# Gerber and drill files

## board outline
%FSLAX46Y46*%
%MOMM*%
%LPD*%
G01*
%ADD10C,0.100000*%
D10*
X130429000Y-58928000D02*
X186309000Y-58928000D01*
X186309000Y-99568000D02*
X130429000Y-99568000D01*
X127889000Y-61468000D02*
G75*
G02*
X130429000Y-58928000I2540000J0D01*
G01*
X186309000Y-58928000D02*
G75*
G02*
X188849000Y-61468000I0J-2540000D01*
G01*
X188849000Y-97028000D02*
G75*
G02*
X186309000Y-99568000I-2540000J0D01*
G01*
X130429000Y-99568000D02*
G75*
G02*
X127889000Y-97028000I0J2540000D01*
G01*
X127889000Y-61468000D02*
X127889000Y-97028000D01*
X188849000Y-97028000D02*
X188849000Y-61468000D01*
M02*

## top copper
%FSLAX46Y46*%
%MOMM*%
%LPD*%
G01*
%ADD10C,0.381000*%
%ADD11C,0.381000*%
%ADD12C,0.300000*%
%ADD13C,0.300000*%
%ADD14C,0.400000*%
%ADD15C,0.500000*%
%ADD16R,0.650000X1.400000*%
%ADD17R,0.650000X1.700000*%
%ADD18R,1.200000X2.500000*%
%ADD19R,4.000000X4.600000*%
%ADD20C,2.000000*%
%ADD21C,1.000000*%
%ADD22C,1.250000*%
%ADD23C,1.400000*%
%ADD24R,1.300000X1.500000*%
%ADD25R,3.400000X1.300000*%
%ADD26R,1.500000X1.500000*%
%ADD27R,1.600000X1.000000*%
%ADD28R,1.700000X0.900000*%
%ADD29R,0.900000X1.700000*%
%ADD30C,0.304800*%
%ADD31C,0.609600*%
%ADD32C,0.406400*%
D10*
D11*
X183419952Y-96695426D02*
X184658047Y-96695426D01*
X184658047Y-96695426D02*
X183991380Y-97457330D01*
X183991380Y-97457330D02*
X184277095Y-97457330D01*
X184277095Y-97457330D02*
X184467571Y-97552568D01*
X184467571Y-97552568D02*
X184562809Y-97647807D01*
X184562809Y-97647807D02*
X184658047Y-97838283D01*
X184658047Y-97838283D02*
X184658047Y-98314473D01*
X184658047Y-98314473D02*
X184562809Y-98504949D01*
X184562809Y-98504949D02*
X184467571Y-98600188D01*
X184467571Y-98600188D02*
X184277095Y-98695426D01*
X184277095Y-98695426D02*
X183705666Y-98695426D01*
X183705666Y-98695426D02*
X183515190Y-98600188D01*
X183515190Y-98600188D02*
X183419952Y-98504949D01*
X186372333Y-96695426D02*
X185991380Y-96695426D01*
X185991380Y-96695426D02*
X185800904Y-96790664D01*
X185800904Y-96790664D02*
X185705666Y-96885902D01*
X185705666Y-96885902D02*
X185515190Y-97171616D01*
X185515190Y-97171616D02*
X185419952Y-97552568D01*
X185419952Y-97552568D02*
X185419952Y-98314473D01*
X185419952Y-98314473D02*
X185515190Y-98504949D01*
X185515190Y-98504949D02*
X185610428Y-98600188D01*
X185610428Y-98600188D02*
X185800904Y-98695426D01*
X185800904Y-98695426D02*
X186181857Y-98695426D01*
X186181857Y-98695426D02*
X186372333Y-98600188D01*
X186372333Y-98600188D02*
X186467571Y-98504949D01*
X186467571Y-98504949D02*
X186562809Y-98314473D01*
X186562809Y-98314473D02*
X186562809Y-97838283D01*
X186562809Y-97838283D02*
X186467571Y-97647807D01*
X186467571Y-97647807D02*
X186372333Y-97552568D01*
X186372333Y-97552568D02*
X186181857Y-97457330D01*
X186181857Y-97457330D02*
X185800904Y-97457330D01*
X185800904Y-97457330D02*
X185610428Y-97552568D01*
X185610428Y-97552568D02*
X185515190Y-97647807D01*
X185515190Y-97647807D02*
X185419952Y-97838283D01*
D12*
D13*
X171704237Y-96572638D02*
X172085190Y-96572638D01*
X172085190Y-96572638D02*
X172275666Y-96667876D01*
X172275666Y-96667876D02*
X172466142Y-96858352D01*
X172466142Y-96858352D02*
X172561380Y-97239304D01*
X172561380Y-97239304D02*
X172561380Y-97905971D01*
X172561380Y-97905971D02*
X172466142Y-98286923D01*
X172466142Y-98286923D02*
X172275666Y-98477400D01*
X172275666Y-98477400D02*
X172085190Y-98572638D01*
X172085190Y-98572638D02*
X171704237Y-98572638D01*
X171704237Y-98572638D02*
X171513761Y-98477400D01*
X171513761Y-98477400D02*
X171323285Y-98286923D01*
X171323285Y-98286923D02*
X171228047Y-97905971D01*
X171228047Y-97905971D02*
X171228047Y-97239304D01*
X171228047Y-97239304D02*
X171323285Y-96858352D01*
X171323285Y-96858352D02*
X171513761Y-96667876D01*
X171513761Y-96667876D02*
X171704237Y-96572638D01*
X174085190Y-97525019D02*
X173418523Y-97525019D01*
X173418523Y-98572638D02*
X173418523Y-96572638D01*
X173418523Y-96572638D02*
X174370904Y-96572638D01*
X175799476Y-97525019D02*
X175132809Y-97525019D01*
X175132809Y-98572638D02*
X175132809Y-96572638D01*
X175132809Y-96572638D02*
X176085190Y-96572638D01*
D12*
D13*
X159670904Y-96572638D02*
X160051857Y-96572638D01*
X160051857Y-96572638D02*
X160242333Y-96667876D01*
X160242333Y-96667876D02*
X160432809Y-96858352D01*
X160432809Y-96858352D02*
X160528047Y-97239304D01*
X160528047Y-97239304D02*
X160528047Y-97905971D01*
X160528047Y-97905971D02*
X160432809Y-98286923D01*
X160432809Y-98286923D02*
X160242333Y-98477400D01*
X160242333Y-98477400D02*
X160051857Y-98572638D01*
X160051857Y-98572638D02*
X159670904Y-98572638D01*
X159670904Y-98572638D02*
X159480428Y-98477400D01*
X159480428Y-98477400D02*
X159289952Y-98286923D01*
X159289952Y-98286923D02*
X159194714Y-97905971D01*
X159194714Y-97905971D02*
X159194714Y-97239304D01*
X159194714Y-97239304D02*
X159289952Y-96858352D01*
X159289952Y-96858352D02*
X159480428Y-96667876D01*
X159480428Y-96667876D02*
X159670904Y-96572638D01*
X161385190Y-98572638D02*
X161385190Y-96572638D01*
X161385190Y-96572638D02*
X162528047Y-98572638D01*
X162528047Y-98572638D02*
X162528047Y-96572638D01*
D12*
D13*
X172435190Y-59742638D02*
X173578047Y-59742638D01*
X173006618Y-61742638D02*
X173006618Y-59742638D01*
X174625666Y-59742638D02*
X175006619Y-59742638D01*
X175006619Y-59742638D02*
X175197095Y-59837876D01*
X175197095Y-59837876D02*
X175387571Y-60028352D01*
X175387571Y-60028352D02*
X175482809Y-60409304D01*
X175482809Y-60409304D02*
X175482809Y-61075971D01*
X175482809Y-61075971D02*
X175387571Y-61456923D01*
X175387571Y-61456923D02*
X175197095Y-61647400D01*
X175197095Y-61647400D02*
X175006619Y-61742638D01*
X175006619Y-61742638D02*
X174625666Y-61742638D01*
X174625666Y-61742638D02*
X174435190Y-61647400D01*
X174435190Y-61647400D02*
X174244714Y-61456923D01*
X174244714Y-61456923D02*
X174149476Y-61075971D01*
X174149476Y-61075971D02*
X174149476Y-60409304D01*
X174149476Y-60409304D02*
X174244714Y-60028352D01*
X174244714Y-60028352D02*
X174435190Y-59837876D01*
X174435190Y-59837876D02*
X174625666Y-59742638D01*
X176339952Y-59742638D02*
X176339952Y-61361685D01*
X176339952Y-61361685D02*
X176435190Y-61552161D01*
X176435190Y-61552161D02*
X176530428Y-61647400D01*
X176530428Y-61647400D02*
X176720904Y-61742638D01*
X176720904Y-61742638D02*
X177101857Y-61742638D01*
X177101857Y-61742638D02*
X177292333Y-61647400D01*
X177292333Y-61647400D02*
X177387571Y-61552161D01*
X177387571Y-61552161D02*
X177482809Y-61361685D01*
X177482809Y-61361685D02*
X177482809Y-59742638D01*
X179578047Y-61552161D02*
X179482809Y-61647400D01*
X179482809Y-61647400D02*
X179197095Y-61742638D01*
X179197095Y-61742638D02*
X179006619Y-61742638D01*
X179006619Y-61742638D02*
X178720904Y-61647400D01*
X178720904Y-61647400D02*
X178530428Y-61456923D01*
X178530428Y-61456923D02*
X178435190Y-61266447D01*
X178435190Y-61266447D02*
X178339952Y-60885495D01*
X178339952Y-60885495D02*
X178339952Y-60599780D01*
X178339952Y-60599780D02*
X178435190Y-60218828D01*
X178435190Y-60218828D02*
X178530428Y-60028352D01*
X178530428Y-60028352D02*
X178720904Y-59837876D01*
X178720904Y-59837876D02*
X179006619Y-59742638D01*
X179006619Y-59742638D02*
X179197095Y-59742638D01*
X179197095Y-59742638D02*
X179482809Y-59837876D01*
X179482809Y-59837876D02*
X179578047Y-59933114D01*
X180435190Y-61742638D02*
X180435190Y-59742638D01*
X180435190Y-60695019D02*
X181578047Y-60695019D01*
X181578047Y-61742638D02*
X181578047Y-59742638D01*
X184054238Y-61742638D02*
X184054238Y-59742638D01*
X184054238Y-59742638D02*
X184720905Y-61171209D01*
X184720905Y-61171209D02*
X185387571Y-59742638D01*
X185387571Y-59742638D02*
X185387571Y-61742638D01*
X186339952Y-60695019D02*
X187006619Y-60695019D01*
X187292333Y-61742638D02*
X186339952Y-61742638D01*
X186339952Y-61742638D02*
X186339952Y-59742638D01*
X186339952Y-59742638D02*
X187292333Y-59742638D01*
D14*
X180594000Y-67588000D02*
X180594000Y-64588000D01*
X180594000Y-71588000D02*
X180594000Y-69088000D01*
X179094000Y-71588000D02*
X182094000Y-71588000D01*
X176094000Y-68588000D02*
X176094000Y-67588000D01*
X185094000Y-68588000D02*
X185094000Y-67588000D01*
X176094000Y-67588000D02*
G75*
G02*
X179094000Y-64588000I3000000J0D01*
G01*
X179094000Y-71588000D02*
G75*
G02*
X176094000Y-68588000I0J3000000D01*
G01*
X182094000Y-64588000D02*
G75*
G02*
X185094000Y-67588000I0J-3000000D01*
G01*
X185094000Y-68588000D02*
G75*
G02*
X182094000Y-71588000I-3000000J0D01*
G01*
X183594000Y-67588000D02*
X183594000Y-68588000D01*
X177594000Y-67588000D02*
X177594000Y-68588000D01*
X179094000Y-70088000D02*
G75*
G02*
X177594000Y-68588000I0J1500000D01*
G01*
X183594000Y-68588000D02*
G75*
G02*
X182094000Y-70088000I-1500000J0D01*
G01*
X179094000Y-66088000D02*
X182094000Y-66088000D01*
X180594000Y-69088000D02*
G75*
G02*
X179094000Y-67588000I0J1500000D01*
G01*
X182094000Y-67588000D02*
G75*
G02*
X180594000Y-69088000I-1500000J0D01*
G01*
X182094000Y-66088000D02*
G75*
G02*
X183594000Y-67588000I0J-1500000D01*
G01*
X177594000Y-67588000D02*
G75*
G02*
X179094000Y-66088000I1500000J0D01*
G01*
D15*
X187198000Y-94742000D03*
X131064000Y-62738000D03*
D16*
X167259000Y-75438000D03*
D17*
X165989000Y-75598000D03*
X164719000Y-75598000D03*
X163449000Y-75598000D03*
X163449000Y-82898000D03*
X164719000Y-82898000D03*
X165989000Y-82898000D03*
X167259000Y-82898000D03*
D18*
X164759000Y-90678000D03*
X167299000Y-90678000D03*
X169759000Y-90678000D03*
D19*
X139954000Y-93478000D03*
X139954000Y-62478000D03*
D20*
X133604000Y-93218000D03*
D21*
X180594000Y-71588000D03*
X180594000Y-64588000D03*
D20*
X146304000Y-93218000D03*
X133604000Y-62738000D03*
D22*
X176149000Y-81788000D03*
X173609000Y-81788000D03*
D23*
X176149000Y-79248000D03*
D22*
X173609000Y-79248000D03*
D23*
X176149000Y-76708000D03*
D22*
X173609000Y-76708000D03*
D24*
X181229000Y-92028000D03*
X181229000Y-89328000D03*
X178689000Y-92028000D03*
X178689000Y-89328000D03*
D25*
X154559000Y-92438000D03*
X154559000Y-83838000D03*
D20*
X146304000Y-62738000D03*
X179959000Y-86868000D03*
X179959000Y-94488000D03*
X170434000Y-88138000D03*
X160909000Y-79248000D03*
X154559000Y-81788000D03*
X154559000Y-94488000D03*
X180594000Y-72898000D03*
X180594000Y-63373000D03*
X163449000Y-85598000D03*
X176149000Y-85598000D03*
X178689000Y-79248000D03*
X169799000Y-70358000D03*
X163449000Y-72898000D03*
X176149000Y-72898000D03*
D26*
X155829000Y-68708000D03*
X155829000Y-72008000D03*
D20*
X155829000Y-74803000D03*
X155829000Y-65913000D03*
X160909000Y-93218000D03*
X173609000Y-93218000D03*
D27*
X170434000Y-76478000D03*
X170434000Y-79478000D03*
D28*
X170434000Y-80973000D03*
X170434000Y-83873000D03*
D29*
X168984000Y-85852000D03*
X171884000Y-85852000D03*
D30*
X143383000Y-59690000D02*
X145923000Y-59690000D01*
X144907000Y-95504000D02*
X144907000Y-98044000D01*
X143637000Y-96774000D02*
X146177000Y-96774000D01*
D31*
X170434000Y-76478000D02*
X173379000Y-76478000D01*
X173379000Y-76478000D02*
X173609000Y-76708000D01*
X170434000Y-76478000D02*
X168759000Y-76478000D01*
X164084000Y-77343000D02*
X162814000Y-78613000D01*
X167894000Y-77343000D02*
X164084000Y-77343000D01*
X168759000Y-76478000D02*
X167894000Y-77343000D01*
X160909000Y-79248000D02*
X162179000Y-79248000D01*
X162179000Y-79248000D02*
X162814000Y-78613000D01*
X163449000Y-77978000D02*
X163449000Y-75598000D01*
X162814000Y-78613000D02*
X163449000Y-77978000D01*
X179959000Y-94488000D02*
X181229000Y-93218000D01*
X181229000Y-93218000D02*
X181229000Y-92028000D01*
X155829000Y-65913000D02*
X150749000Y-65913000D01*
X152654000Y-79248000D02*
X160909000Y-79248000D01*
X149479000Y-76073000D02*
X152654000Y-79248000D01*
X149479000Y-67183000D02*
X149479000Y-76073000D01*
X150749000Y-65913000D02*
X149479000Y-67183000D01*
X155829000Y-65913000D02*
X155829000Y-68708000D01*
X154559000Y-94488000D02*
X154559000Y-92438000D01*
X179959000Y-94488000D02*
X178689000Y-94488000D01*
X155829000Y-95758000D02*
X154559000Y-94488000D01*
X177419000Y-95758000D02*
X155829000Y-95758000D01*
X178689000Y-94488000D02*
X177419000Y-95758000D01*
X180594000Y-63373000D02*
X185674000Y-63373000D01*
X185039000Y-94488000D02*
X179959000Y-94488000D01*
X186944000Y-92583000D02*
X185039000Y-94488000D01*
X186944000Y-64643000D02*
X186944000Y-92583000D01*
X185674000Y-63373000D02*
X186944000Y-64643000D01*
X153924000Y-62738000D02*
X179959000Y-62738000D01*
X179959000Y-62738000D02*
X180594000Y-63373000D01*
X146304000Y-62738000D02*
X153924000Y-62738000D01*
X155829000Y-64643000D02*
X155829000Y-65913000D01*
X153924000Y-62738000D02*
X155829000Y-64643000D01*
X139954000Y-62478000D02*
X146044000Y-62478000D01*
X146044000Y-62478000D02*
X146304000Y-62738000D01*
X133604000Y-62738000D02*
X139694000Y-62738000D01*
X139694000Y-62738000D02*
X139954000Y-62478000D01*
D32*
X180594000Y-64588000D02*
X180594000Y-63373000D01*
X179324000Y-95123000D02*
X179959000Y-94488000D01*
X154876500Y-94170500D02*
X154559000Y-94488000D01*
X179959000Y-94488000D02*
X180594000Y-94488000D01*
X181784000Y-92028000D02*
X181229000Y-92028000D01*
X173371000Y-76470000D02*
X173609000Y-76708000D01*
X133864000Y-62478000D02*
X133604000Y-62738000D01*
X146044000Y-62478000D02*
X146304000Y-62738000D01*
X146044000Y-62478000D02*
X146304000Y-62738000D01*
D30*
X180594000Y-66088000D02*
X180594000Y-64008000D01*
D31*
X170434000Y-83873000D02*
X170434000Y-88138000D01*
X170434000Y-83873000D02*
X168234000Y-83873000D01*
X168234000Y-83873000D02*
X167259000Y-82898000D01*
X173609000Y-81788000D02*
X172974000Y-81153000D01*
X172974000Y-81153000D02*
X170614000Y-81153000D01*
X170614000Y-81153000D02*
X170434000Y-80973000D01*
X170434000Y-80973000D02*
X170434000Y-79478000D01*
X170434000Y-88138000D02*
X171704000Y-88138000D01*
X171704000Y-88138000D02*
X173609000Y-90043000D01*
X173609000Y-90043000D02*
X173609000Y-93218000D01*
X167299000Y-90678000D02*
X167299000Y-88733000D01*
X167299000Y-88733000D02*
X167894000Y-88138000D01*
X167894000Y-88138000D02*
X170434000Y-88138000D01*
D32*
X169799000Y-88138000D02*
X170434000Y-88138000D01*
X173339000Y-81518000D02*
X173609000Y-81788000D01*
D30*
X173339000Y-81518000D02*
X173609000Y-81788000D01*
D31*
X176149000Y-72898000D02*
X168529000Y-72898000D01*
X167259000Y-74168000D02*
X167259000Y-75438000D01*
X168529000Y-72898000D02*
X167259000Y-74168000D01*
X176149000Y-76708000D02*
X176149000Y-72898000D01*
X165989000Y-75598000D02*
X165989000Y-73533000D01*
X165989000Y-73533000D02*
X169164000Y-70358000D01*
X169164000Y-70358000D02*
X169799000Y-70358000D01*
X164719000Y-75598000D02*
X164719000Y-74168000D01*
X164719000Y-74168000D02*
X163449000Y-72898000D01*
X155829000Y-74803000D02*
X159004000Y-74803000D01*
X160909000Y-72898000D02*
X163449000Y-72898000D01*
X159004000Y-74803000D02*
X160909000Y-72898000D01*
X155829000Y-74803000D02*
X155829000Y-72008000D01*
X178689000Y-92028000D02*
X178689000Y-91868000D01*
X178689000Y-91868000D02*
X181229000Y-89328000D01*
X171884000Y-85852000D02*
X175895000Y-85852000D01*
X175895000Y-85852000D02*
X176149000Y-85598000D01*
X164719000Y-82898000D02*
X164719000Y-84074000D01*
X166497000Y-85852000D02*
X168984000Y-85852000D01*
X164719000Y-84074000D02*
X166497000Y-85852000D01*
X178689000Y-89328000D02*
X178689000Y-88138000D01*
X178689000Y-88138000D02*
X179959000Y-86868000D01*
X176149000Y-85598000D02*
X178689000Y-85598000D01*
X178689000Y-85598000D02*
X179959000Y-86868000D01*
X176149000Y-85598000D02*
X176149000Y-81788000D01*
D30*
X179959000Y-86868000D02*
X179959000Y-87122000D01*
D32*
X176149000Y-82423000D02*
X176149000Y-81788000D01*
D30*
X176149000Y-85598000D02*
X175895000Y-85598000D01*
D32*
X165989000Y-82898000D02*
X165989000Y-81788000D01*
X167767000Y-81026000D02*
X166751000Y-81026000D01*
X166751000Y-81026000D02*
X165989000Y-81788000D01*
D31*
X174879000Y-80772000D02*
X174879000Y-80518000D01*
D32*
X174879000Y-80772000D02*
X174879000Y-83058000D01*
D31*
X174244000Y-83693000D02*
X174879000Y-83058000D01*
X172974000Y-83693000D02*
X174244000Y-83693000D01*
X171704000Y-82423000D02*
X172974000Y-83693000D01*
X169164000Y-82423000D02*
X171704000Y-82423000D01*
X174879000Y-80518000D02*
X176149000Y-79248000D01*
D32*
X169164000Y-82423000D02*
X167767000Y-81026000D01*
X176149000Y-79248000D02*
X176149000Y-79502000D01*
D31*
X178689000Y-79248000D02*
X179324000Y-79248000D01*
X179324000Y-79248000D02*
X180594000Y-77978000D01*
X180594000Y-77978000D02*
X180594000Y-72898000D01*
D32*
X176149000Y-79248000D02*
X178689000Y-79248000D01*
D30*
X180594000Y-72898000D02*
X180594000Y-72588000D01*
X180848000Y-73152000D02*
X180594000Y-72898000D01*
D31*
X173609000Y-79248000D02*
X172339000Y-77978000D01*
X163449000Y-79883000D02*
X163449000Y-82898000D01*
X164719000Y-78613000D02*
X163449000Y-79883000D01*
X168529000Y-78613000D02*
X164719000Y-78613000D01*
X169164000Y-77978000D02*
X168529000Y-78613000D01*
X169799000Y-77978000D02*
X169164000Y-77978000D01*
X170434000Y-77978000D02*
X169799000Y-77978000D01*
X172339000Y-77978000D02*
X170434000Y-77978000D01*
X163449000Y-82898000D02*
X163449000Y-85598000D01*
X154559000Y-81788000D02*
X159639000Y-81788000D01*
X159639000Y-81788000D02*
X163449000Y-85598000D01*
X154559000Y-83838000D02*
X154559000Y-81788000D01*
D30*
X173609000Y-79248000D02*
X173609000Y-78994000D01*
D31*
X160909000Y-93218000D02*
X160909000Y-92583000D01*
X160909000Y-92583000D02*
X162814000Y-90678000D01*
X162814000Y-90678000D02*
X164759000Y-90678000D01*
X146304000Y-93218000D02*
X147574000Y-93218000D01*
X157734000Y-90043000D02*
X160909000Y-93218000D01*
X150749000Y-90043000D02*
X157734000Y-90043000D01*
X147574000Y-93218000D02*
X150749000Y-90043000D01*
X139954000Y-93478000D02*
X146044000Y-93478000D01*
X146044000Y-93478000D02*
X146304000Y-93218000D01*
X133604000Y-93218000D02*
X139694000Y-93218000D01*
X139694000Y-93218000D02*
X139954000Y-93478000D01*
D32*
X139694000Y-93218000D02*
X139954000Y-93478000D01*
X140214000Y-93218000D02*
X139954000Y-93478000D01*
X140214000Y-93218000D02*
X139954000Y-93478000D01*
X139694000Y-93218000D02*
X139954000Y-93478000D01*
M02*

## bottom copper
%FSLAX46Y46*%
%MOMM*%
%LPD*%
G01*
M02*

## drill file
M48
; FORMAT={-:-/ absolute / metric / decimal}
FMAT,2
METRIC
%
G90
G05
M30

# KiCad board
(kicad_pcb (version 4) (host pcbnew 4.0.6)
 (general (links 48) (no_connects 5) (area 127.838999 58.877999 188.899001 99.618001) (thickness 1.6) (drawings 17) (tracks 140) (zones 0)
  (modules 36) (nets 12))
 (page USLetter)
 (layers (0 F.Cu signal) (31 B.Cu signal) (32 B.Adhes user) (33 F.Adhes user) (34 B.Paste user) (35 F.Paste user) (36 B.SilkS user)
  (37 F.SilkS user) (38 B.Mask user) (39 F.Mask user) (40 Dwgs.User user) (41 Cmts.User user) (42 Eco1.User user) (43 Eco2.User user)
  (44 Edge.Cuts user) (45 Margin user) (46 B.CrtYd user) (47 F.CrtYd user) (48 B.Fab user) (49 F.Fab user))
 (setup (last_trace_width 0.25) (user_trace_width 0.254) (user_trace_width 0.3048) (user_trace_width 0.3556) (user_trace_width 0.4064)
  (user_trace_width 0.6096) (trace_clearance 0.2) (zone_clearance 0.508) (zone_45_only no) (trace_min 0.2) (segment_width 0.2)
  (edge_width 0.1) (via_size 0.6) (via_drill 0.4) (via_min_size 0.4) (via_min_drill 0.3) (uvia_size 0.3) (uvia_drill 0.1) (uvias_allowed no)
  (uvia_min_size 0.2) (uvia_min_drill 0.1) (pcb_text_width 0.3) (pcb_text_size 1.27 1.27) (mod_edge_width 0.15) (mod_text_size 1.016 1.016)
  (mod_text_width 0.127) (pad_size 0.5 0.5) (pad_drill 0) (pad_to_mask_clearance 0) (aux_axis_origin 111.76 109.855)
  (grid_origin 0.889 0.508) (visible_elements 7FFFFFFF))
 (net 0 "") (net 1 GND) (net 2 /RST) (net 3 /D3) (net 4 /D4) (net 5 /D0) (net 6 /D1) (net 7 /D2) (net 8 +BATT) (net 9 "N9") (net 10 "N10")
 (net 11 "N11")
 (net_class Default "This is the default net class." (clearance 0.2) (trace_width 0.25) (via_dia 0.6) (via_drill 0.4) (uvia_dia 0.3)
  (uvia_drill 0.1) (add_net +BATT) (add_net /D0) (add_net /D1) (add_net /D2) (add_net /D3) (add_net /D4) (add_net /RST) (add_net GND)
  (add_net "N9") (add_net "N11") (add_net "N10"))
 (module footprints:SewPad (layer F.Cu) (at 187.198 94.742)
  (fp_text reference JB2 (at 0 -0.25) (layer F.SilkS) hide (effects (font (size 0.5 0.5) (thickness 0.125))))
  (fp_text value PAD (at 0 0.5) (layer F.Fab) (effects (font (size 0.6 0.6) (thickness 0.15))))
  (pad 1 smd circle (at 0 0) (size 0.5 0.5) (layers F.Cu F.Mask) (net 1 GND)))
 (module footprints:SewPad (layer F.Cu) (at 131.064 62.738)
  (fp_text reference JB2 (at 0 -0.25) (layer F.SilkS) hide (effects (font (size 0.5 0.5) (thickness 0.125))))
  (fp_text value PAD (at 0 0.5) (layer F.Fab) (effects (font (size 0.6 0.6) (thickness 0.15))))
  (pad 1 smd circle (at 0 0) (size 0.5 0.5) (layers F.Cu F.Mask) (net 1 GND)))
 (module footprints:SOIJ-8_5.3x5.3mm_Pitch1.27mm (layer F.Cu) (at 165.354 79.248 270)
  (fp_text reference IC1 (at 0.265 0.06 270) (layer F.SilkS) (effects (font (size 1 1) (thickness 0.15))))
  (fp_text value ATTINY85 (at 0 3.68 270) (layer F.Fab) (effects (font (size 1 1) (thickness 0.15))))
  (pad 1 smd rect (at -3.81 -1.905 270) (size 1.4 0.65) (layers F.Cu F.Paste F.Mask) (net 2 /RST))
  (pad 2 smd rect (at -3.65 -0.635 270) (size 1.7 0.65) (layers F.Cu F.Paste F.Mask) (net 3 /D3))
  (pad 3 smd rect (at -3.65 0.635 270) (size 1.7 0.65) (layers F.Cu F.Paste F.Mask) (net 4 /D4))
  (pad 4 smd rect (at -3.65 1.905 270) (size 1.7 0.65) (layers F.Cu F.Paste F.Mask) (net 1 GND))
  (pad 5 smd rect (at 3.65 1.905 270) (size 1.7 0.65) (layers F.Cu F.Paste F.Mask) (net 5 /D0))
  (pad 6 smd rect (at 3.65 0.635 270) (size 1.7 0.65) (layers F.Cu F.Paste F.Mask) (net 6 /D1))
  (pad 7 smd rect (at 3.65 -0.635 270) (size 1.7 0.65) (layers F.Cu F.Paste F.Mask) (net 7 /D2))
  (pad 8 smd rect (at 3.65 -1.905 270) (size 1.7 0.65) (layers F.Cu F.Paste F.Mask) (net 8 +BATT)))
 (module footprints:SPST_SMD (layer F.Cu) (at 167.259 90.678)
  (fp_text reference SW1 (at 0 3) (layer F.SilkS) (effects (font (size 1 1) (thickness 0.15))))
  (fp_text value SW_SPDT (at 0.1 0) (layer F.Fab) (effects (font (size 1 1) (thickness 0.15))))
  (pad 1 smd rect (at -2.5 0) (size 1.2 2.5) (layers F.Cu F.Paste F.Mask) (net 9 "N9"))
  (pad 2 smd rect (at 0.04 0) (size 1.2 2.5) (layers F.Cu F.Paste F.Mask) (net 8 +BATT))
  (pad 3 smd rect (at 2.5 0) (size 1.2 2.5) (layers F.Cu F.Paste F.Mask) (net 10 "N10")))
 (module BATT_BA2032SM (layer F.Cu) (at 139.954 77.978 90)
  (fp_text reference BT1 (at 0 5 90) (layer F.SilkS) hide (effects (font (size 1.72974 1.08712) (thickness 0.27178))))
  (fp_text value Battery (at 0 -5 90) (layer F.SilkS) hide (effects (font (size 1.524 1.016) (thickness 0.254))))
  (pad 1 smd rect (at -15.5 0 90) (size 4.6 4) (layers F.Cu F.Paste F.Mask) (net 9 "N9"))
  (pad 2 smd rect (at 15.5 0 90) (size 4.6 4) (layers F.Cu F.Paste F.Mask) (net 1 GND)))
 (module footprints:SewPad (layer F.Cu) (at 133.604 93.218)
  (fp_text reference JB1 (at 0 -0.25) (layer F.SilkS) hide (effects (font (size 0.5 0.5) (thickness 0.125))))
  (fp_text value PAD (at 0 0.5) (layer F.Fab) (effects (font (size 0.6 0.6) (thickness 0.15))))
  (pad 1 smd circle (at 0 0) (size 2 2) (layers F.Cu F.Mask) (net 9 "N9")))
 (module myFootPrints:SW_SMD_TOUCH (layer F.Cu) (at 180.594 69.088)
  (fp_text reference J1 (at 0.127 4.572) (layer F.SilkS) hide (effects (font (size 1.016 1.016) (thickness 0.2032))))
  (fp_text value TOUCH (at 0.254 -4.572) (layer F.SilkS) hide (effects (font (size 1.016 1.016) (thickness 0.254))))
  (fp_line (start 0 -1.5) (end 0 -4.5) (layer F.Cu) (width 0.4)) (fp_line (start 0 2.5) (end 0 0) (layer F.Cu) (width 0.4))
  (fp_line (start -1.5 2.5) (end 1.5 2.5) (layer F.Cu) (width 0.4))
  (fp_line (start -4.5 -0.5) (end -4.5 -1.5) (layer F.Cu) (width 0.4))
  (fp_line (start 4.5 -0.5) (end 4.5 -1.5) (layer F.Cu) (width 0.4))
  (fp_arc (start -1.5 -1.5) (end -4.5 -1.5) (angle 90) (layer F.Cu) (width 0.4))
  (fp_arc (start -1.5 -0.5) (end -1.5 2.5) (angle 90) (layer F.Cu) (width 0.4))
  (fp_arc (start 1.5 -1.5) (end 1.5 -4.5) (angle 90) (layer F.Cu) (width 0.4))
  (fp_arc (start 1.5 -0.5) (end 4.5 -0.5) (angle 90) (layer F.Cu) (width 0.4))
  (fp_line (start 3 -1.5) (end 3 -0.5) (layer F.Cu) (width 0.4))
  (fp_line (start -3 -1.5) (end -3 -0.5) (layer F.Cu) (width 0.4))
  (fp_arc (start -1.5 -0.5) (end -1.5 1) (angle 90) (layer F.Cu) (width 0.4))
  (fp_arc (start 1.5 -0.5) (end 3 -0.5) (angle 90) (layer F.Cu) (width 0.4))
  (fp_line (start -1.5 -3) (end 1.5 -3) (layer F.Cu) (width 0.4))
  (fp_arc (start 0 -1.5) (end 0 0) (angle 90) (layer F.Cu) (width 0.4))
  (fp_arc (start 0 -1.5) (end 1.5 -1.5) (angle 90) (layer F.Cu) (width 0.4))
  (fp_arc (start 1.5 -1.5) (end 1.5 -3) (angle 90) (layer F.Cu) (width 0.4))
  (fp_arc (start -1.5 -1.5) (end -3 -1.5) (angle 90) (layer F.Cu) (width 0.4))
  (pad 2 smd circle (at 0 2.5) (size 1 1) (layers F.Cu) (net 7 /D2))
  (pad 1 smd circle (at 0 -4.5) (size 1 1) (layers F.Cu) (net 1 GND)))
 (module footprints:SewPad (layer F.Cu) (at 146.304 93.218)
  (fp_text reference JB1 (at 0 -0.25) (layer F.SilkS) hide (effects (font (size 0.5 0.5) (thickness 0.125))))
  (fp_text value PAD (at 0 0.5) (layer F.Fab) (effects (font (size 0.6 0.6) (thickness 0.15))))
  (pad 1 smd circle (at 0 0) (size 2 2) (layers F.Cu F.Mask) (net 9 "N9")))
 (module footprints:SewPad (layer F.Cu) (at 133.604 62.738)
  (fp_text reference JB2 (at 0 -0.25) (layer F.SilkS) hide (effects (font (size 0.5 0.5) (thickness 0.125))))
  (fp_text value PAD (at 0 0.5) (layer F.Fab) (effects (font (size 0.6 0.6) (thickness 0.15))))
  (pad 1 smd circle (at 0 0) (size 2 2) (layers F.Cu F.Mask) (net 1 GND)))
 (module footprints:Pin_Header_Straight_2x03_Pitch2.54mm (layer F.Cu) (at 176.149 81.788 180)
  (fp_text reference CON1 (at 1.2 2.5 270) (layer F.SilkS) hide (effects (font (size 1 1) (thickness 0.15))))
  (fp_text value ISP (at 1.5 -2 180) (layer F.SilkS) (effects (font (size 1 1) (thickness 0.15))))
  (pad 1 smd circle (at 0 0 180) (size 1.25 1.25) (layers F.Cu) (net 6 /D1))
  (pad 2 smd circle (at 2.54 0 180) (size 1.25 1.25) (layers F.Cu) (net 8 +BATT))
  (pad 3 smd circle (at 0 2.54 180) (size 1.4 1.4) (layers F.Cu) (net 7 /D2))
  (pad 4 smd circle (at 2.54 2.54 180) (size 1.25 1.25) (layers F.Cu) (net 5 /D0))
  (pad 5 smd circle (at 0 5.08 180) (size 1.4 1.4) (layers F.Cu) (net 2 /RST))
  (pad 6 smd circle (at 2.54 5.08 180) (size 1.25 1.25) (layers F.Cu) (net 1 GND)))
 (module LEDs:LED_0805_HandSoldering (layer F.Cu) (at 181.229 90.678 90)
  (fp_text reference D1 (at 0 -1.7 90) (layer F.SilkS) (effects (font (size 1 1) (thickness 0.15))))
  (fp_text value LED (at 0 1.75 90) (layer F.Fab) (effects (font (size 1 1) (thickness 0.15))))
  (pad 1 smd rect (at -1.35 0 90) (size 1.5 1.3) (layers F.Cu F.Paste F.Mask) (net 1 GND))
  (pad 2 smd rect (at 1.35 0 90) (size 1.5 1.3) (layers F.Cu F.Paste F.Mask) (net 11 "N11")))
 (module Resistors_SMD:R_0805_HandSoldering (layer F.Cu) (at 178.689 90.678 90)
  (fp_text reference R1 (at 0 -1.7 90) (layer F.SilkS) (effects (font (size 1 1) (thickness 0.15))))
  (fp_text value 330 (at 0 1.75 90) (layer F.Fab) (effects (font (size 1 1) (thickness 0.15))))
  (pad 1 smd rect (at -1.35 0 90) (size 1.5 1.3) (layers F.Cu F.Paste F.Mask) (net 11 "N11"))
  (pad 2 smd rect (at 1.35 0 90) (size 1.5 1.3) (layers F.Cu F.Paste F.Mask) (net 6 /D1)))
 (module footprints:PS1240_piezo (layer F.Cu) (at 154.559 88.138 90)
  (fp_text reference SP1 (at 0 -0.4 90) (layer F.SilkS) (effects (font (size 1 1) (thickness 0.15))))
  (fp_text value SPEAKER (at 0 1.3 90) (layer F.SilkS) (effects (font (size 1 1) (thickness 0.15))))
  (pad 1 smd rect (at -4.3 0 90) (size 1.3 3.4) (layers F.Cu F.Paste F.Mask) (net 1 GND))
  (pad 2 smd rect (at 4.3 0 90) (size 1.3 3.4) (layers F.Cu F.Paste F.Mask) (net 5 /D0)))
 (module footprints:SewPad (layer F.Cu) (at 146.304 62.738)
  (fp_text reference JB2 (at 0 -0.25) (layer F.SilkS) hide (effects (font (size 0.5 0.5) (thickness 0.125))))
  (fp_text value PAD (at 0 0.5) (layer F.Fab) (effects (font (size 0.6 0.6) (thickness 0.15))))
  (pad 1 smd circle (at 0 0) (size 2 2) (layers F.Cu F.Mask) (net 1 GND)))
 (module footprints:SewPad (layer F.Cu) (at 179.959 86.868 90)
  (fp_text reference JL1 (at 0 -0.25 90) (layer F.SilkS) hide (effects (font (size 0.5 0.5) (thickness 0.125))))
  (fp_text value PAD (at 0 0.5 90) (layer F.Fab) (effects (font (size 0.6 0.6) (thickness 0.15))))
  (pad 1 smd circle (at 0 0 90) (size 2 2) (layers F.Cu F.Mask) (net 6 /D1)))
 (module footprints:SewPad (layer F.Cu) (at 179.959 94.488 90)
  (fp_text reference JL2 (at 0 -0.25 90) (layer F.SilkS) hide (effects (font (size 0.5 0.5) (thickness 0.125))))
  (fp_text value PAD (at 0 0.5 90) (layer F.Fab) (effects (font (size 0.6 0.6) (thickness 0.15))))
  (pad 1 smd circle (at 0 0 90) (size 2 2) (layers F.Cu F.Mask) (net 1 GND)))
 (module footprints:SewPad (layer F.Cu) (at 170.434 88.138)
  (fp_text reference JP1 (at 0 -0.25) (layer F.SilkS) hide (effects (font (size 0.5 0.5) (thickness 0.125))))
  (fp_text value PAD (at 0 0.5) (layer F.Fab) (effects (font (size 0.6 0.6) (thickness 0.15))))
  (pad 1 smd circle (at 0 0) (size 2 2) (layers F.Cu F.Mask) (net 8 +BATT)))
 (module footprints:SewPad (layer F.Cu) (at 160.909 79.248)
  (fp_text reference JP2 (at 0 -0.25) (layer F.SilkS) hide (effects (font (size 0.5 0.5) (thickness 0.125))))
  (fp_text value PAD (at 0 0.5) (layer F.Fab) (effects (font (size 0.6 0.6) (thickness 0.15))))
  (pad 1 smd circle (at 0 0) (size 2 2) (layers F.Cu F.Mask) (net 1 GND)))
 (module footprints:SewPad (layer F.Cu) (at 154.559 81.788 180)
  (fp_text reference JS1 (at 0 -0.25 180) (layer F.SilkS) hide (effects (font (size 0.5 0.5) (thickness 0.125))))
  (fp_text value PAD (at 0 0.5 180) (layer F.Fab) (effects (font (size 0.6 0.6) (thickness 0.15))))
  (pad 1 smd circle (at 0 0 180) (size 2 2) (layers F.Cu F.Mask) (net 5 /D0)))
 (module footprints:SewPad (layer F.Cu) (at 154.559 94.488 180)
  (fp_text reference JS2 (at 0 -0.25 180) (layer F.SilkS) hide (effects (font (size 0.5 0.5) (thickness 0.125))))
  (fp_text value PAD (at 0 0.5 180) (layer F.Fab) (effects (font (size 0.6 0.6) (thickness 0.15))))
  (pad 1 smd circle (at 0 0 180) (size 2 2) (layers F.Cu F.Mask) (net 1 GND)))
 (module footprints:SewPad (layer F.Cu) (at 180.594 72.898 90)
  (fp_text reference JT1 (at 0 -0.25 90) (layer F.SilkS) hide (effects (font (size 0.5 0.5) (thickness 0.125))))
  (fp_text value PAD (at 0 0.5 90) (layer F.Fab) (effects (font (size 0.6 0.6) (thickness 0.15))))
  (pad 1 smd circle (at 0 0 90) (size 2 2) (layers F.Cu F.Mask) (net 7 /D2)))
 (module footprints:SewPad (layer F.Cu) (at 180.594 63.373 90)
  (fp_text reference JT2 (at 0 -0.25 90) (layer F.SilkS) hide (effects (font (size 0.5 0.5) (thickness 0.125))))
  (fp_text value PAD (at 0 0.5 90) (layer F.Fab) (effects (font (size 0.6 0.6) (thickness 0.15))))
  (pad 1 smd circle (at 0 0 90) (size 2 2) (layers F.Cu F.Mask) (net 1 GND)))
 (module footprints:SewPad (layer F.Cu) (at 163.449 85.598)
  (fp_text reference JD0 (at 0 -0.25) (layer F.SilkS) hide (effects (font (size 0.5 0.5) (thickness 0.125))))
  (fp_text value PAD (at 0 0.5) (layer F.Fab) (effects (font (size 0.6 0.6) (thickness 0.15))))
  (pad 1 smd circle (at 0 0) (size 2 2) (layers F.Cu F.Mask) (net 5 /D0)))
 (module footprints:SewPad (layer F.Cu) (at 176.149 85.598)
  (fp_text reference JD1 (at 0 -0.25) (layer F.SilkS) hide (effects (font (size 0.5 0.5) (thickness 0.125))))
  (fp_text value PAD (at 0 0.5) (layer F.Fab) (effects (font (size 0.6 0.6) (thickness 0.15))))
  (pad 1 smd circle (at 0 0) (size 2 2) (layers F.Cu F.Mask) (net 6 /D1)))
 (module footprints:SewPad (layer F.Cu) (at 178.689 79.248)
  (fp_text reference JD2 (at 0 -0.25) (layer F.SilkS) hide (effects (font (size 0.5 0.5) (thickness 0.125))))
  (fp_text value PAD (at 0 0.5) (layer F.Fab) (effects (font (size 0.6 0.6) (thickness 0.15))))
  (pad 1 smd circle (at 0 0) (size 2 2) (layers F.Cu F.Mask) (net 7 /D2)))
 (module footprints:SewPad (layer F.Cu) (at 169.799 70.358)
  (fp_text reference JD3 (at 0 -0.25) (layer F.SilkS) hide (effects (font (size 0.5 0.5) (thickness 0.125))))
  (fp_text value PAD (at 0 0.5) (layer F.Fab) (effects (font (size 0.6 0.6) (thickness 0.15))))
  (pad 1 smd circle (at 0 0) (size 2 2) (layers F.Cu F.Mask) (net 3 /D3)))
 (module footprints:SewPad (layer F.Cu) (at 163.449 72.898)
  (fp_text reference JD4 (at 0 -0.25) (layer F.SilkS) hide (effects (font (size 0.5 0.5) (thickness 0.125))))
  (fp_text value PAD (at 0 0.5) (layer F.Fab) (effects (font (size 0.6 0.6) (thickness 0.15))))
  (pad 1 smd circle (at 0 0) (size 2 2) (layers F.Cu F.Mask) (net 4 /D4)))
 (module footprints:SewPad (layer F.Cu) (at 176.149 72.898)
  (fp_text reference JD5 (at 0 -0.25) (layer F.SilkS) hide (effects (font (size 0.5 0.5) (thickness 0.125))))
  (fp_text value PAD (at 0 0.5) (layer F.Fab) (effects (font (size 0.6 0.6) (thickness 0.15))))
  (pad 1 smd circle (at 0 0) (size 2 2) (layers F.Cu F.Mask) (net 2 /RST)))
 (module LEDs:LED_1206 (layer F.Cu) (at 155.829 70.358 90)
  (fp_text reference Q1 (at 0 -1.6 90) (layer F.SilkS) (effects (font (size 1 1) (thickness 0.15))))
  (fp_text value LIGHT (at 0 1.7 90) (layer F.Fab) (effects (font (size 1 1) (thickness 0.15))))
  (pad 2 smd rect (at 1.65 0 270) (size 1.5 1.5) (layers F.Cu F.Paste F.Mask) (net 1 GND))
  (pad 1 smd rect (at -1.65 0 270) (size 1.5 1.5) (layers F.Cu F.Paste F.Mask) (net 4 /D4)))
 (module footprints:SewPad (layer F.Cu) (at 155.829 74.803)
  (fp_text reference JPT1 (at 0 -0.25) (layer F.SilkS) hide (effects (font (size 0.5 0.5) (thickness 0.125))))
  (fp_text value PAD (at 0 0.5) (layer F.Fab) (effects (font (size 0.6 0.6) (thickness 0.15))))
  (pad 1 smd circle (at 0 0) (size 2 2) (layers F.Cu F.Mask) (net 4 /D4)))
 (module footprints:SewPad (layer F.Cu) (at 155.829 65.913)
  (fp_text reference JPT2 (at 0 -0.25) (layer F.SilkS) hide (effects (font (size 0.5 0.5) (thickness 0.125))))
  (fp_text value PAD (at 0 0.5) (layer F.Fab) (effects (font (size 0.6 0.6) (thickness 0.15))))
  (pad 1 smd circle (at 0 0) (size 2 2) (layers F.Cu F.Mask) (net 1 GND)))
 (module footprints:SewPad (layer F.Cu) (at 160.909 93.218)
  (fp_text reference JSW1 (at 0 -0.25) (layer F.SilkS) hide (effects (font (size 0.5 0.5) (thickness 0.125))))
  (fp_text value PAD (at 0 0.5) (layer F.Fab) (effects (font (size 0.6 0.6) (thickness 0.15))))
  (pad 1 smd circle (at 0 0) (size 2 2) (layers F.Cu F.Mask) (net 9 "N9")))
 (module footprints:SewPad (layer F.Cu) (at 173.609 93.218)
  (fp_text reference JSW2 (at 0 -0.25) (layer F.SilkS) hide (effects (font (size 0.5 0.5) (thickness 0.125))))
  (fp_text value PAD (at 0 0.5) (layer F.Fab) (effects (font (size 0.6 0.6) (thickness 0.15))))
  (pad 1 smd circle (at 0 0) (size 2 2) (layers F.Cu F.Mask) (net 8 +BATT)))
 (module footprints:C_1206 (layer F.Cu) (at 170.434 77.978 270)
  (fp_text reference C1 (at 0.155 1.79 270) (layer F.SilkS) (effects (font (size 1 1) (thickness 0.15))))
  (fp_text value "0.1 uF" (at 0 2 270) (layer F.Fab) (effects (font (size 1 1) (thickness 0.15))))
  (pad 1 smd rect (at -1.5 0 270) (size 1 1.6) (layers F.Cu F.Paste F.Mask) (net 1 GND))
  (pad 2 smd rect (at 1.5 0 270) (size 1 1.6) (layers F.Cu F.Paste F.Mask) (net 8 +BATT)))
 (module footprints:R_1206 (layer F.Cu) (at 170.434 82.423 270)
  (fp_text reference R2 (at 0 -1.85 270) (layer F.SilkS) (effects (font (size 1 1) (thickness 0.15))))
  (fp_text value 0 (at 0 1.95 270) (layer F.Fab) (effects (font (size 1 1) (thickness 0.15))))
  (pad 1 smd rect (at -1.45 0 270) (size 0.9 1.7) (layers F.Cu F.Paste F.Mask) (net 8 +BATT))
  (pad 2 smd rect (at 1.45 0 270) (size 0.9 1.7) (layers F.Cu F.Paste F.Mask) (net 8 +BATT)))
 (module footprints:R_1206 (layer F.Cu) (at 170.434 85.852)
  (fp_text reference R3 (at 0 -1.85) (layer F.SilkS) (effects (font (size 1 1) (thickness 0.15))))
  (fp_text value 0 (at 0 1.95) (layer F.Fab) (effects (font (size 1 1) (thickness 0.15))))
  (pad 1 smd rect (at -1.45 0) (size 0.9 1.7) (layers F.Cu F.Paste F.Mask) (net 6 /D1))
  (pad 2 smd rect (at 1.45 0) (size 0.9 1.7) (layers F.Cu F.Paste F.Mask) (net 6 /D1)))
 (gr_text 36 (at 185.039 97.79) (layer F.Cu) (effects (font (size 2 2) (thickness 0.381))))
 (gr_line (start 130.429 58.928) (end 186.309 58.928) (angle 90) (layer Edge.Cuts) (width 0.1))
 (gr_line (start 186.309 99.568) (end 130.429 99.568) (angle 90) (layer Edge.Cuts) (width 0.1))
 (gr_arc (start 130.429 61.468) (end 127.889 61.468) (angle 90) (layer Edge.Cuts) (width 0.1))
 (gr_arc (start 186.309 61.468) (end 186.309 58.928) (angle 90) (layer Edge.Cuts) (width 0.1))
 (gr_arc (start 186.309 97.028) (end 188.849 97.028) (angle 90) (layer Edge.Cuts) (width 0.1))
 (gr_arc (start 130.429 97.028) (end 130.429 99.568) (angle 90) (layer Edge.Cuts) (width 0.1))
 (gr_line (start 127.889 61.468) (end 127.889 97.028) (angle 90) (layer Edge.Cuts) (width 0.1))
 (gr_line (start 188.849 97.028) (end 188.849 61.468) (angle 90) (layer Edge.Cuts) (width 0.1))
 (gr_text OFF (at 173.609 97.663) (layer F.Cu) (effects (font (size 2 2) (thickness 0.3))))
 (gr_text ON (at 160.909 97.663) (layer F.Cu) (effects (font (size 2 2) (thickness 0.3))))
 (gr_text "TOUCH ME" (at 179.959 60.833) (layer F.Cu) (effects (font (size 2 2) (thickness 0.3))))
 (segment (start 143.383 59.69) (end 145.923 59.69) (width 0.3048) (layer F.Cu) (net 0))
 (segment (start 144.907 95.504) (end 144.907 98.044) (width 0.3048) (layer F.Cu) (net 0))
 (segment (start 143.637 96.774) (end 146.177 96.774) (width 0.3048) (layer F.Cu) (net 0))
 (segment (start 170.434 76.478) (end 173.379 76.478) (width 0.6096) (layer F.Cu) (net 1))
 (segment (start 173.379 76.478) (end 173.609 76.708) (width 0.6096) (layer F.Cu) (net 1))
 (segment (start 170.434 76.478) (end 168.759 76.478) (width 0.6096) (layer F.Cu) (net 1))
 (segment (start 164.084 77.343) (end 162.814 78.613) (width 0.6096) (layer F.Cu) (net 1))
 (segment (start 167.894 77.343) (end 164.084 77.343) (width 0.6096) (layer F.Cu) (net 1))
 (segment (start 168.759 76.478) (end 167.894 77.343) (width 0.6096) (layer F.Cu) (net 1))
 (segment (start 160.909 79.248) (end 162.179 79.248) (width 0.6096) (layer F.Cu) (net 1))
 (segment (start 162.179 79.248) (end 162.814 78.613) (width 0.6096) (layer F.Cu) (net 1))
 (segment (start 163.449 77.978) (end 163.449 75.598) (width 0.6096) (layer F.Cu) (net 1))
 (segment (start 162.814 78.613) (end 163.449 77.978) (width 0.6096) (layer F.Cu) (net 1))
 (segment (start 179.959 94.488) (end 181.229 93.218) (width 0.6096) (layer F.Cu) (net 1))
 (segment (start 181.229 93.218) (end 181.229 92.028) (width 0.6096) (layer F.Cu) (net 1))
 (segment (start 155.829 65.913) (end 150.749 65.913) (width 0.6096) (layer F.Cu) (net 1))
 (segment (start 152.654 79.248) (end 160.909 79.248) (width 0.6096) (layer F.Cu) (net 1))
 (segment (start 149.479 76.073) (end 152.654 79.248) (width 0.6096) (layer F.Cu) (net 1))
 (segment (start 149.479 67.183) (end 149.479 76.073) (width 0.6096) (layer F.Cu) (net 1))
 (segment (start 150.749 65.913) (end 149.479 67.183) (width 0.6096) (layer F.Cu) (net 1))
 (segment (start 155.829 65.913) (end 155.829 68.708) (width 0.6096) (layer F.Cu) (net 1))
 (segment (start 154.559 94.488) (end 154.559 92.438) (width 0.6096) (layer F.Cu) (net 1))
 (segment (start 179.959 94.488) (end 178.689 94.488) (width 0.6096) (layer F.Cu) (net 1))
 (segment (start 155.829 95.758) (end 154.559 94.488) (width 0.6096) (layer F.Cu) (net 1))
 (segment (start 177.419 95.758) (end 155.829 95.758) (width 0.6096) (layer F.Cu) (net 1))
 (segment (start 178.689 94.488) (end 177.419 95.758) (width 0.6096) (layer F.Cu) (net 1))
 (segment (start 180.594 63.373) (end 185.674 63.373) (width 0.6096) (layer F.Cu) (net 1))
 (segment (start 185.039 94.488) (end 179.959 94.488) (width 0.6096) (layer F.Cu) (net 1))
 (segment (start 186.944 92.583) (end 185.039 94.488) (width 0.6096) (layer F.Cu) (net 1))
 (segment (start 186.944 64.643) (end 186.944 92.583) (width 0.6096) (layer F.Cu) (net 1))
 (segment (start 185.674 63.373) (end 186.944 64.643) (width 0.6096) (layer F.Cu) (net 1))
 (segment (start 153.924 62.738) (end 179.959 62.738) (width 0.6096) (layer F.Cu) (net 1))
 (segment (start 179.959 62.738) (end 180.594 63.373) (width 0.6096) (layer F.Cu) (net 1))
 (segment (start 146.304 62.738) (end 153.924 62.738) (width 0.6096) (layer F.Cu) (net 1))
 (segment (start 155.829 64.643) (end 155.829 65.913) (width 0.6096) (layer F.Cu) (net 1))
 (segment (start 153.924 62.738) (end 155.829 64.643) (width 0.6096) (layer F.Cu) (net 1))
 (segment (start 139.954 62.478) (end 146.044 62.478) (width 0.6096) (layer F.Cu) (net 1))
 (segment (start 146.044 62.478) (end 146.304 62.738) (width 0.6096) (layer F.Cu) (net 1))
 (segment (start 133.604 62.738) (end 139.694 62.738) (width 0.6096) (layer F.Cu) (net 1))
 (segment (start 139.694 62.738) (end 139.954 62.478) (width 0.6096) (layer F.Cu) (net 1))
 (segment (start 180.594 64.588) (end 180.594 63.373) (width 0.4064) (layer F.Cu) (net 1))
 (segment (start 179.324 95.123) (end 179.959 94.488) (width 0.4064) (layer F.Cu) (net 1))
 (segment (start 154.8765 94.1705) (end 154.559 94.488) (width 0.4064) (layer F.Cu) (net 1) (status 30))
 (segment (start 179.959 94.488) (end 180.594 94.488) (width 0.4064) (layer F.Cu) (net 1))
 (segment (start 181.784 92.028) (end 181.229 92.028) (width 0.4064) (layer F.Cu) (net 1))
 (segment (start 173.371 76.47) (end 173.609 76.708) (width 0.4064) (layer F.Cu) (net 1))
 (segment (start 133.864 62.478) (end 133.604 62.738) (width 0.4064) (layer F.Cu) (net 1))
 (segment (start 146.044 62.478) (end 146.304 62.738) (width 0.4064) (layer F.Cu) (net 1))
 (segment (start 146.044 62.478) (end 146.304 62.738) (width 0.4064) (layer F.Cu) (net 1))
 (segment (start 180.594 66.088) (end 180.594 64.008) (width 0.3048) (layer F.Cu) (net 1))
 (segment (start 170.434 83.873) (end 170.434 88.138) (width 0.6096) (layer F.Cu) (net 8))
 (segment (start 170.434 83.873) (end 168.234 83.873) (width 0.6096) (layer F.Cu) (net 8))
 (segment (start 168.234 83.873) (end 167.259 82.898) (width 0.6096) (layer F.Cu) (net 8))
 (segment (start 173.609 81.788) (end 172.974 81.153) (width 0.6096) (layer F.Cu) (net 8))
 (segment (start 172.974 81.153) (end 170.614 81.153) (width 0.6096) (layer F.Cu) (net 8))
 (segment (start 170.614 81.153) (end 170.434 80.973) (width 0.6096) (layer F.Cu) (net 8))
 (segment (start 170.434 80.973) (end 170.434 79.478) (width 0.6096) (layer F.Cu) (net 8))
 (segment (start 170.434 88.138) (end 171.704 88.138) (width 0.6096) (layer F.Cu) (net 8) (status 10))
 (segment (start 171.704 88.138) (end 173.609 90.043) (width 0.6096) (layer F.Cu) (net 8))
 (segment (start 173.609 90.043) (end 173.609 93.218) (width 0.6096) (layer F.Cu) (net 8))
 (segment (start 167.299 90.678) (end 167.299 88.733) (width 0.6096) (layer F.Cu) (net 8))
 (segment (start 167.299 88.733) (end 167.894 88.138) (width 0.6096) (layer F.Cu) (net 8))
 (segment (start 167.894 88.138) (end 170.434 88.138) (width 0.6096) (layer F.Cu) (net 8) (status 20))
 (segment (start 169.799 88.138) (end 170.434 88.138) (width 0.4064) (layer F.Cu) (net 8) (status 30))
 (segment (start 173.339 81.518) (end 173.609 81.788) (width 0.4064) (layer F.Cu) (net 8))
 (segment (start 173.339 81.518) (end 173.609 81.788) (width 0.3048) (layer F.Cu) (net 8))
 (segment (start 176.149 72.898) (end 168.529 72.898) (width 0.6096) (layer F.Cu) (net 2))
 (segment (start 167.259 74.168) (end 167.259 75.438) (width 0.6096) (layer F.Cu) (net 2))
 (segment (start 168.529 72.898) (end 167.259 74.168) (width 0.6096) (layer F.Cu) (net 2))
 (segment (start 176.149 76.708) (end 176.149 72.898) (width 0.6096) (layer F.Cu) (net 2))
 (segment (start 165.989 75.598) (end 165.989 73.533) (width 0.6096) (layer F.Cu) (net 3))
 (segment (start 165.989 73.533) (end 169.164 70.358) (width 0.6096) (layer F.Cu) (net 3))
 (segment (start 169.164 70.358) (end 169.799 70.358) (width 0.6096) (layer F.Cu) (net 3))
 (segment (start 164.719 75.598) (end 164.719 74.168) (width 0.6096) (layer F.Cu) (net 4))
 (segment (start 164.719 74.168) (end 163.449 72.898) (width 0.6096) (layer F.Cu) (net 4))
 (segment (start 155.829 74.803) (end 159.004 74.803) (width 0.6096) (layer F.Cu) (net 4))
 (segment (start 160.909 72.898) (end 163.449 72.898) (width 0.6096) (layer F.Cu) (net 4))
 (segment (start 159.004 74.803) (end 160.909 72.898) (width 0.6096) (layer F.Cu) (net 4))
 (segment (start 155.829 74.803) (end 155.829 72.008) (width 0.6096) (layer F.Cu) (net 4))
 (segment (start 178.689 92.028) (end 178.689 91.868) (width 0.6096) (layer F.Cu) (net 11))
 (segment (start 178.689 91.868) (end 181.229 89.328) (width 0.6096) (layer F.Cu) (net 11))
 (segment (start 171.884 85.852) (end 175.895 85.852) (width 0.6096) (layer F.Cu) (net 6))
 (segment (start 175.895 85.852) (end 176.149 85.598) (width 0.6096) (layer F.Cu) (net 6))
 (segment (start 164.719 82.898) (end 164.719 84.074) (width 0.6096) (layer F.Cu) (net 6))
 (segment (start 166.497 85.852) (end 168.984 85.852) (width 0.6096) (layer F.Cu) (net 6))
 (segment (start 164.719 84.074) (end 166.497 85.852) (width 0.6096) (layer F.Cu) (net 6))
 (segment (start 178.689 89.328) (end 178.689 88.138) (width 0.6096) (layer F.Cu) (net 6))
 (segment (start 178.689 88.138) (end 179.959 86.868) (width 0.6096) (layer F.Cu) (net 6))
 (segment (start 176.149 85.598) (end 178.689 85.598) (width 0.6096) (layer F.Cu) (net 6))
 (segment (start 178.689 85.598) (end 179.959 86.868) (width 0.6096) (layer F.Cu) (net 6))
 (segment (start 176.149 85.598) (end 176.149 81.788) (width 0.6096) (layer F.Cu) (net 6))
 (segment (start 179.959 86.868) (end 179.959 87.122) (width 0.3048) (layer F.Cu) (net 6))
 (segment (start 176.149 82.423) (end 176.149 81.788) (width 0.4064) (layer F.Cu) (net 6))
 (segment (start 176.149 85.598) (end 175.895 85.598) (width 0.3048) (layer F.Cu) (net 6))
 (segment (start 165.989 82.898) (end 165.989 81.788) (width 0.4064) (layer F.Cu) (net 7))
 (segment (start 167.767 81.026) (end 166.751 81.026) (width 0.4064) (layer F.Cu) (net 7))
 (segment (start 166.751 81.026) (end 165.989 81.788) (width 0.4064) (layer F.Cu) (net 7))
 (segment (start 174.879 80.772) (end 174.879 80.518) (width 0.6096) (layer F.Cu) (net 7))
 (segment (start 174.879 80.772) (end 174.879 83.058) (width 0.4064) (layer F.Cu) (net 7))
 (segment (start 174.244 83.693) (end 174.879 83.058) (width 0.6096) (layer F.Cu) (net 7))
 (segment (start 172.974 83.693) (end 174.244 83.693) (width 0.6096) (layer F.Cu) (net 7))
 (segment (start 171.704 82.423) (end 172.974 83.693) (width 0.6096) (layer F.Cu) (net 7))
 (segment (start 169.164 82.423) (end 171.704 82.423) (width 0.6096) (layer F.Cu) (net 7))
 (segment (start 174.879 80.518) (end 176.149 79.248) (width 0.6096) (layer F.Cu) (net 7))
 (segment (start 169.164 82.423) (end 167.767 81.026) (width 0.4064) (layer F.Cu) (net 7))
 (segment (start 176.149 79.248) (end 176.149 79.502) (width 0.4064) (layer F.Cu) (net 7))
 (segment (start 178.689 79.248) (end 179.324 79.248) (width 0.6096) (layer F.Cu) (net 7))
 (segment (start 179.324 79.248) (end 180.594 77.978) (width 0.6096) (layer F.Cu) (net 7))
 (segment (start 180.594 77.978) (end 180.594 72.898) (width 0.6096) (layer F.Cu) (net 7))
 (segment (start 176.149 79.248) (end 178.689 79.248) (width 0.4064) (layer F.Cu) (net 7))
 (segment (start 180.594 72.898) (end 180.594 72.588) (width 0.3048) (layer F.Cu) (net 7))
 (segment (start 180.848 73.152) (end 180.594 72.898) (width 0.3048) (layer F.Cu) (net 7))
 (segment (start 173.609 79.248) (end 172.339 77.978) (width 0.6096) (layer F.Cu) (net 5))
 (segment (start 163.449 79.883) (end 163.449 82.898) (width 0.6096) (layer F.Cu) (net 5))
 (segment (start 164.719 78.613) (end 163.449 79.883) (width 0.6096) (layer F.Cu) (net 5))
 (segment (start 168.529 78.613) (end 164.719 78.613) (width 0.6096) (layer F.Cu) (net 5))
 (segment (start 169.164 77.978) (end 168.529 78.613) (width 0.6096) (layer F.Cu) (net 5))
 (segment (start 169.799 77.978) (end 169.164 77.978) (width 0.6096) (layer F.Cu) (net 5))
 (segment (start 170.434 77.978) (end 169.799 77.978) (width 0.6096) (layer F.Cu) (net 5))
 (segment (start 172.339 77.978) (end 170.434 77.978) (width 0.6096) (layer F.Cu) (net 5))
 (segment (start 163.449 82.898) (end 163.449 85.598) (width 0.6096) (layer F.Cu) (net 5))
 (segment (start 154.559 81.788) (end 159.639 81.788) (width 0.6096) (layer F.Cu) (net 5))
 (segment (start 159.639 81.788) (end 163.449 85.598) (width 0.6096) (layer F.Cu) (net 5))
 (segment (start 154.559 83.838) (end 154.559 81.788) (width 0.6096) (layer F.Cu) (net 5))
 (segment (start 173.609 79.248) (end 173.609 78.994) (width 0.3048) (layer F.Cu) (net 5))
 (segment (start 160.909 93.218) (end 160.909 92.583) (width 0.6096) (layer F.Cu) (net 9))
 (segment (start 160.909 92.583) (end 162.814 90.678) (width 0.6096) (layer F.Cu) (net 9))
 (segment (start 162.814 90.678) (end 164.759 90.678) (width 0.6096) (layer F.Cu) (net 9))
 (segment (start 146.304 93.218) (end 147.574 93.218) (width 0.6096) (layer F.Cu) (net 9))
 (segment (start 157.734 90.043) (end 160.909 93.218) (width 0.6096) (layer F.Cu) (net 9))
 (segment (start 150.749 90.043) (end 157.734 90.043) (width 0.6096) (layer F.Cu) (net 9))
 (segment (start 147.574 93.218) (end 150.749 90.043) (width 0.6096) (layer F.Cu) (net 9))
 (segment (start 139.954 93.478) (end 146.044 93.478) (width 0.6096) (layer F.Cu) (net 9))
 (segment (start 146.044 93.478) (end 146.304 93.218) (width 0.6096) (layer F.Cu) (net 9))
 (segment (start 133.604 93.218) (end 139.694 93.218) (width 0.6096) (layer F.Cu) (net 9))
 (segment (start 139.694 93.218) (end 139.954 93.478) (width 0.6096) (layer F.Cu) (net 9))
 (segment (start 139.694 93.218) (end 139.954 93.478) (width 0.4064) (layer F.Cu) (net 9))
 (segment (start 140.214 93.218) (end 139.954 93.478) (width 0.4064) (layer F.Cu) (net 9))
 (segment (start 140.214 93.218) (end 139.954 93.478) (width 0.4064) (layer F.Cu) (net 9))
 (segment (start 139.694 93.218) (end 139.954 93.478) (width 0.4064) (layer F.Cu) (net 9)))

